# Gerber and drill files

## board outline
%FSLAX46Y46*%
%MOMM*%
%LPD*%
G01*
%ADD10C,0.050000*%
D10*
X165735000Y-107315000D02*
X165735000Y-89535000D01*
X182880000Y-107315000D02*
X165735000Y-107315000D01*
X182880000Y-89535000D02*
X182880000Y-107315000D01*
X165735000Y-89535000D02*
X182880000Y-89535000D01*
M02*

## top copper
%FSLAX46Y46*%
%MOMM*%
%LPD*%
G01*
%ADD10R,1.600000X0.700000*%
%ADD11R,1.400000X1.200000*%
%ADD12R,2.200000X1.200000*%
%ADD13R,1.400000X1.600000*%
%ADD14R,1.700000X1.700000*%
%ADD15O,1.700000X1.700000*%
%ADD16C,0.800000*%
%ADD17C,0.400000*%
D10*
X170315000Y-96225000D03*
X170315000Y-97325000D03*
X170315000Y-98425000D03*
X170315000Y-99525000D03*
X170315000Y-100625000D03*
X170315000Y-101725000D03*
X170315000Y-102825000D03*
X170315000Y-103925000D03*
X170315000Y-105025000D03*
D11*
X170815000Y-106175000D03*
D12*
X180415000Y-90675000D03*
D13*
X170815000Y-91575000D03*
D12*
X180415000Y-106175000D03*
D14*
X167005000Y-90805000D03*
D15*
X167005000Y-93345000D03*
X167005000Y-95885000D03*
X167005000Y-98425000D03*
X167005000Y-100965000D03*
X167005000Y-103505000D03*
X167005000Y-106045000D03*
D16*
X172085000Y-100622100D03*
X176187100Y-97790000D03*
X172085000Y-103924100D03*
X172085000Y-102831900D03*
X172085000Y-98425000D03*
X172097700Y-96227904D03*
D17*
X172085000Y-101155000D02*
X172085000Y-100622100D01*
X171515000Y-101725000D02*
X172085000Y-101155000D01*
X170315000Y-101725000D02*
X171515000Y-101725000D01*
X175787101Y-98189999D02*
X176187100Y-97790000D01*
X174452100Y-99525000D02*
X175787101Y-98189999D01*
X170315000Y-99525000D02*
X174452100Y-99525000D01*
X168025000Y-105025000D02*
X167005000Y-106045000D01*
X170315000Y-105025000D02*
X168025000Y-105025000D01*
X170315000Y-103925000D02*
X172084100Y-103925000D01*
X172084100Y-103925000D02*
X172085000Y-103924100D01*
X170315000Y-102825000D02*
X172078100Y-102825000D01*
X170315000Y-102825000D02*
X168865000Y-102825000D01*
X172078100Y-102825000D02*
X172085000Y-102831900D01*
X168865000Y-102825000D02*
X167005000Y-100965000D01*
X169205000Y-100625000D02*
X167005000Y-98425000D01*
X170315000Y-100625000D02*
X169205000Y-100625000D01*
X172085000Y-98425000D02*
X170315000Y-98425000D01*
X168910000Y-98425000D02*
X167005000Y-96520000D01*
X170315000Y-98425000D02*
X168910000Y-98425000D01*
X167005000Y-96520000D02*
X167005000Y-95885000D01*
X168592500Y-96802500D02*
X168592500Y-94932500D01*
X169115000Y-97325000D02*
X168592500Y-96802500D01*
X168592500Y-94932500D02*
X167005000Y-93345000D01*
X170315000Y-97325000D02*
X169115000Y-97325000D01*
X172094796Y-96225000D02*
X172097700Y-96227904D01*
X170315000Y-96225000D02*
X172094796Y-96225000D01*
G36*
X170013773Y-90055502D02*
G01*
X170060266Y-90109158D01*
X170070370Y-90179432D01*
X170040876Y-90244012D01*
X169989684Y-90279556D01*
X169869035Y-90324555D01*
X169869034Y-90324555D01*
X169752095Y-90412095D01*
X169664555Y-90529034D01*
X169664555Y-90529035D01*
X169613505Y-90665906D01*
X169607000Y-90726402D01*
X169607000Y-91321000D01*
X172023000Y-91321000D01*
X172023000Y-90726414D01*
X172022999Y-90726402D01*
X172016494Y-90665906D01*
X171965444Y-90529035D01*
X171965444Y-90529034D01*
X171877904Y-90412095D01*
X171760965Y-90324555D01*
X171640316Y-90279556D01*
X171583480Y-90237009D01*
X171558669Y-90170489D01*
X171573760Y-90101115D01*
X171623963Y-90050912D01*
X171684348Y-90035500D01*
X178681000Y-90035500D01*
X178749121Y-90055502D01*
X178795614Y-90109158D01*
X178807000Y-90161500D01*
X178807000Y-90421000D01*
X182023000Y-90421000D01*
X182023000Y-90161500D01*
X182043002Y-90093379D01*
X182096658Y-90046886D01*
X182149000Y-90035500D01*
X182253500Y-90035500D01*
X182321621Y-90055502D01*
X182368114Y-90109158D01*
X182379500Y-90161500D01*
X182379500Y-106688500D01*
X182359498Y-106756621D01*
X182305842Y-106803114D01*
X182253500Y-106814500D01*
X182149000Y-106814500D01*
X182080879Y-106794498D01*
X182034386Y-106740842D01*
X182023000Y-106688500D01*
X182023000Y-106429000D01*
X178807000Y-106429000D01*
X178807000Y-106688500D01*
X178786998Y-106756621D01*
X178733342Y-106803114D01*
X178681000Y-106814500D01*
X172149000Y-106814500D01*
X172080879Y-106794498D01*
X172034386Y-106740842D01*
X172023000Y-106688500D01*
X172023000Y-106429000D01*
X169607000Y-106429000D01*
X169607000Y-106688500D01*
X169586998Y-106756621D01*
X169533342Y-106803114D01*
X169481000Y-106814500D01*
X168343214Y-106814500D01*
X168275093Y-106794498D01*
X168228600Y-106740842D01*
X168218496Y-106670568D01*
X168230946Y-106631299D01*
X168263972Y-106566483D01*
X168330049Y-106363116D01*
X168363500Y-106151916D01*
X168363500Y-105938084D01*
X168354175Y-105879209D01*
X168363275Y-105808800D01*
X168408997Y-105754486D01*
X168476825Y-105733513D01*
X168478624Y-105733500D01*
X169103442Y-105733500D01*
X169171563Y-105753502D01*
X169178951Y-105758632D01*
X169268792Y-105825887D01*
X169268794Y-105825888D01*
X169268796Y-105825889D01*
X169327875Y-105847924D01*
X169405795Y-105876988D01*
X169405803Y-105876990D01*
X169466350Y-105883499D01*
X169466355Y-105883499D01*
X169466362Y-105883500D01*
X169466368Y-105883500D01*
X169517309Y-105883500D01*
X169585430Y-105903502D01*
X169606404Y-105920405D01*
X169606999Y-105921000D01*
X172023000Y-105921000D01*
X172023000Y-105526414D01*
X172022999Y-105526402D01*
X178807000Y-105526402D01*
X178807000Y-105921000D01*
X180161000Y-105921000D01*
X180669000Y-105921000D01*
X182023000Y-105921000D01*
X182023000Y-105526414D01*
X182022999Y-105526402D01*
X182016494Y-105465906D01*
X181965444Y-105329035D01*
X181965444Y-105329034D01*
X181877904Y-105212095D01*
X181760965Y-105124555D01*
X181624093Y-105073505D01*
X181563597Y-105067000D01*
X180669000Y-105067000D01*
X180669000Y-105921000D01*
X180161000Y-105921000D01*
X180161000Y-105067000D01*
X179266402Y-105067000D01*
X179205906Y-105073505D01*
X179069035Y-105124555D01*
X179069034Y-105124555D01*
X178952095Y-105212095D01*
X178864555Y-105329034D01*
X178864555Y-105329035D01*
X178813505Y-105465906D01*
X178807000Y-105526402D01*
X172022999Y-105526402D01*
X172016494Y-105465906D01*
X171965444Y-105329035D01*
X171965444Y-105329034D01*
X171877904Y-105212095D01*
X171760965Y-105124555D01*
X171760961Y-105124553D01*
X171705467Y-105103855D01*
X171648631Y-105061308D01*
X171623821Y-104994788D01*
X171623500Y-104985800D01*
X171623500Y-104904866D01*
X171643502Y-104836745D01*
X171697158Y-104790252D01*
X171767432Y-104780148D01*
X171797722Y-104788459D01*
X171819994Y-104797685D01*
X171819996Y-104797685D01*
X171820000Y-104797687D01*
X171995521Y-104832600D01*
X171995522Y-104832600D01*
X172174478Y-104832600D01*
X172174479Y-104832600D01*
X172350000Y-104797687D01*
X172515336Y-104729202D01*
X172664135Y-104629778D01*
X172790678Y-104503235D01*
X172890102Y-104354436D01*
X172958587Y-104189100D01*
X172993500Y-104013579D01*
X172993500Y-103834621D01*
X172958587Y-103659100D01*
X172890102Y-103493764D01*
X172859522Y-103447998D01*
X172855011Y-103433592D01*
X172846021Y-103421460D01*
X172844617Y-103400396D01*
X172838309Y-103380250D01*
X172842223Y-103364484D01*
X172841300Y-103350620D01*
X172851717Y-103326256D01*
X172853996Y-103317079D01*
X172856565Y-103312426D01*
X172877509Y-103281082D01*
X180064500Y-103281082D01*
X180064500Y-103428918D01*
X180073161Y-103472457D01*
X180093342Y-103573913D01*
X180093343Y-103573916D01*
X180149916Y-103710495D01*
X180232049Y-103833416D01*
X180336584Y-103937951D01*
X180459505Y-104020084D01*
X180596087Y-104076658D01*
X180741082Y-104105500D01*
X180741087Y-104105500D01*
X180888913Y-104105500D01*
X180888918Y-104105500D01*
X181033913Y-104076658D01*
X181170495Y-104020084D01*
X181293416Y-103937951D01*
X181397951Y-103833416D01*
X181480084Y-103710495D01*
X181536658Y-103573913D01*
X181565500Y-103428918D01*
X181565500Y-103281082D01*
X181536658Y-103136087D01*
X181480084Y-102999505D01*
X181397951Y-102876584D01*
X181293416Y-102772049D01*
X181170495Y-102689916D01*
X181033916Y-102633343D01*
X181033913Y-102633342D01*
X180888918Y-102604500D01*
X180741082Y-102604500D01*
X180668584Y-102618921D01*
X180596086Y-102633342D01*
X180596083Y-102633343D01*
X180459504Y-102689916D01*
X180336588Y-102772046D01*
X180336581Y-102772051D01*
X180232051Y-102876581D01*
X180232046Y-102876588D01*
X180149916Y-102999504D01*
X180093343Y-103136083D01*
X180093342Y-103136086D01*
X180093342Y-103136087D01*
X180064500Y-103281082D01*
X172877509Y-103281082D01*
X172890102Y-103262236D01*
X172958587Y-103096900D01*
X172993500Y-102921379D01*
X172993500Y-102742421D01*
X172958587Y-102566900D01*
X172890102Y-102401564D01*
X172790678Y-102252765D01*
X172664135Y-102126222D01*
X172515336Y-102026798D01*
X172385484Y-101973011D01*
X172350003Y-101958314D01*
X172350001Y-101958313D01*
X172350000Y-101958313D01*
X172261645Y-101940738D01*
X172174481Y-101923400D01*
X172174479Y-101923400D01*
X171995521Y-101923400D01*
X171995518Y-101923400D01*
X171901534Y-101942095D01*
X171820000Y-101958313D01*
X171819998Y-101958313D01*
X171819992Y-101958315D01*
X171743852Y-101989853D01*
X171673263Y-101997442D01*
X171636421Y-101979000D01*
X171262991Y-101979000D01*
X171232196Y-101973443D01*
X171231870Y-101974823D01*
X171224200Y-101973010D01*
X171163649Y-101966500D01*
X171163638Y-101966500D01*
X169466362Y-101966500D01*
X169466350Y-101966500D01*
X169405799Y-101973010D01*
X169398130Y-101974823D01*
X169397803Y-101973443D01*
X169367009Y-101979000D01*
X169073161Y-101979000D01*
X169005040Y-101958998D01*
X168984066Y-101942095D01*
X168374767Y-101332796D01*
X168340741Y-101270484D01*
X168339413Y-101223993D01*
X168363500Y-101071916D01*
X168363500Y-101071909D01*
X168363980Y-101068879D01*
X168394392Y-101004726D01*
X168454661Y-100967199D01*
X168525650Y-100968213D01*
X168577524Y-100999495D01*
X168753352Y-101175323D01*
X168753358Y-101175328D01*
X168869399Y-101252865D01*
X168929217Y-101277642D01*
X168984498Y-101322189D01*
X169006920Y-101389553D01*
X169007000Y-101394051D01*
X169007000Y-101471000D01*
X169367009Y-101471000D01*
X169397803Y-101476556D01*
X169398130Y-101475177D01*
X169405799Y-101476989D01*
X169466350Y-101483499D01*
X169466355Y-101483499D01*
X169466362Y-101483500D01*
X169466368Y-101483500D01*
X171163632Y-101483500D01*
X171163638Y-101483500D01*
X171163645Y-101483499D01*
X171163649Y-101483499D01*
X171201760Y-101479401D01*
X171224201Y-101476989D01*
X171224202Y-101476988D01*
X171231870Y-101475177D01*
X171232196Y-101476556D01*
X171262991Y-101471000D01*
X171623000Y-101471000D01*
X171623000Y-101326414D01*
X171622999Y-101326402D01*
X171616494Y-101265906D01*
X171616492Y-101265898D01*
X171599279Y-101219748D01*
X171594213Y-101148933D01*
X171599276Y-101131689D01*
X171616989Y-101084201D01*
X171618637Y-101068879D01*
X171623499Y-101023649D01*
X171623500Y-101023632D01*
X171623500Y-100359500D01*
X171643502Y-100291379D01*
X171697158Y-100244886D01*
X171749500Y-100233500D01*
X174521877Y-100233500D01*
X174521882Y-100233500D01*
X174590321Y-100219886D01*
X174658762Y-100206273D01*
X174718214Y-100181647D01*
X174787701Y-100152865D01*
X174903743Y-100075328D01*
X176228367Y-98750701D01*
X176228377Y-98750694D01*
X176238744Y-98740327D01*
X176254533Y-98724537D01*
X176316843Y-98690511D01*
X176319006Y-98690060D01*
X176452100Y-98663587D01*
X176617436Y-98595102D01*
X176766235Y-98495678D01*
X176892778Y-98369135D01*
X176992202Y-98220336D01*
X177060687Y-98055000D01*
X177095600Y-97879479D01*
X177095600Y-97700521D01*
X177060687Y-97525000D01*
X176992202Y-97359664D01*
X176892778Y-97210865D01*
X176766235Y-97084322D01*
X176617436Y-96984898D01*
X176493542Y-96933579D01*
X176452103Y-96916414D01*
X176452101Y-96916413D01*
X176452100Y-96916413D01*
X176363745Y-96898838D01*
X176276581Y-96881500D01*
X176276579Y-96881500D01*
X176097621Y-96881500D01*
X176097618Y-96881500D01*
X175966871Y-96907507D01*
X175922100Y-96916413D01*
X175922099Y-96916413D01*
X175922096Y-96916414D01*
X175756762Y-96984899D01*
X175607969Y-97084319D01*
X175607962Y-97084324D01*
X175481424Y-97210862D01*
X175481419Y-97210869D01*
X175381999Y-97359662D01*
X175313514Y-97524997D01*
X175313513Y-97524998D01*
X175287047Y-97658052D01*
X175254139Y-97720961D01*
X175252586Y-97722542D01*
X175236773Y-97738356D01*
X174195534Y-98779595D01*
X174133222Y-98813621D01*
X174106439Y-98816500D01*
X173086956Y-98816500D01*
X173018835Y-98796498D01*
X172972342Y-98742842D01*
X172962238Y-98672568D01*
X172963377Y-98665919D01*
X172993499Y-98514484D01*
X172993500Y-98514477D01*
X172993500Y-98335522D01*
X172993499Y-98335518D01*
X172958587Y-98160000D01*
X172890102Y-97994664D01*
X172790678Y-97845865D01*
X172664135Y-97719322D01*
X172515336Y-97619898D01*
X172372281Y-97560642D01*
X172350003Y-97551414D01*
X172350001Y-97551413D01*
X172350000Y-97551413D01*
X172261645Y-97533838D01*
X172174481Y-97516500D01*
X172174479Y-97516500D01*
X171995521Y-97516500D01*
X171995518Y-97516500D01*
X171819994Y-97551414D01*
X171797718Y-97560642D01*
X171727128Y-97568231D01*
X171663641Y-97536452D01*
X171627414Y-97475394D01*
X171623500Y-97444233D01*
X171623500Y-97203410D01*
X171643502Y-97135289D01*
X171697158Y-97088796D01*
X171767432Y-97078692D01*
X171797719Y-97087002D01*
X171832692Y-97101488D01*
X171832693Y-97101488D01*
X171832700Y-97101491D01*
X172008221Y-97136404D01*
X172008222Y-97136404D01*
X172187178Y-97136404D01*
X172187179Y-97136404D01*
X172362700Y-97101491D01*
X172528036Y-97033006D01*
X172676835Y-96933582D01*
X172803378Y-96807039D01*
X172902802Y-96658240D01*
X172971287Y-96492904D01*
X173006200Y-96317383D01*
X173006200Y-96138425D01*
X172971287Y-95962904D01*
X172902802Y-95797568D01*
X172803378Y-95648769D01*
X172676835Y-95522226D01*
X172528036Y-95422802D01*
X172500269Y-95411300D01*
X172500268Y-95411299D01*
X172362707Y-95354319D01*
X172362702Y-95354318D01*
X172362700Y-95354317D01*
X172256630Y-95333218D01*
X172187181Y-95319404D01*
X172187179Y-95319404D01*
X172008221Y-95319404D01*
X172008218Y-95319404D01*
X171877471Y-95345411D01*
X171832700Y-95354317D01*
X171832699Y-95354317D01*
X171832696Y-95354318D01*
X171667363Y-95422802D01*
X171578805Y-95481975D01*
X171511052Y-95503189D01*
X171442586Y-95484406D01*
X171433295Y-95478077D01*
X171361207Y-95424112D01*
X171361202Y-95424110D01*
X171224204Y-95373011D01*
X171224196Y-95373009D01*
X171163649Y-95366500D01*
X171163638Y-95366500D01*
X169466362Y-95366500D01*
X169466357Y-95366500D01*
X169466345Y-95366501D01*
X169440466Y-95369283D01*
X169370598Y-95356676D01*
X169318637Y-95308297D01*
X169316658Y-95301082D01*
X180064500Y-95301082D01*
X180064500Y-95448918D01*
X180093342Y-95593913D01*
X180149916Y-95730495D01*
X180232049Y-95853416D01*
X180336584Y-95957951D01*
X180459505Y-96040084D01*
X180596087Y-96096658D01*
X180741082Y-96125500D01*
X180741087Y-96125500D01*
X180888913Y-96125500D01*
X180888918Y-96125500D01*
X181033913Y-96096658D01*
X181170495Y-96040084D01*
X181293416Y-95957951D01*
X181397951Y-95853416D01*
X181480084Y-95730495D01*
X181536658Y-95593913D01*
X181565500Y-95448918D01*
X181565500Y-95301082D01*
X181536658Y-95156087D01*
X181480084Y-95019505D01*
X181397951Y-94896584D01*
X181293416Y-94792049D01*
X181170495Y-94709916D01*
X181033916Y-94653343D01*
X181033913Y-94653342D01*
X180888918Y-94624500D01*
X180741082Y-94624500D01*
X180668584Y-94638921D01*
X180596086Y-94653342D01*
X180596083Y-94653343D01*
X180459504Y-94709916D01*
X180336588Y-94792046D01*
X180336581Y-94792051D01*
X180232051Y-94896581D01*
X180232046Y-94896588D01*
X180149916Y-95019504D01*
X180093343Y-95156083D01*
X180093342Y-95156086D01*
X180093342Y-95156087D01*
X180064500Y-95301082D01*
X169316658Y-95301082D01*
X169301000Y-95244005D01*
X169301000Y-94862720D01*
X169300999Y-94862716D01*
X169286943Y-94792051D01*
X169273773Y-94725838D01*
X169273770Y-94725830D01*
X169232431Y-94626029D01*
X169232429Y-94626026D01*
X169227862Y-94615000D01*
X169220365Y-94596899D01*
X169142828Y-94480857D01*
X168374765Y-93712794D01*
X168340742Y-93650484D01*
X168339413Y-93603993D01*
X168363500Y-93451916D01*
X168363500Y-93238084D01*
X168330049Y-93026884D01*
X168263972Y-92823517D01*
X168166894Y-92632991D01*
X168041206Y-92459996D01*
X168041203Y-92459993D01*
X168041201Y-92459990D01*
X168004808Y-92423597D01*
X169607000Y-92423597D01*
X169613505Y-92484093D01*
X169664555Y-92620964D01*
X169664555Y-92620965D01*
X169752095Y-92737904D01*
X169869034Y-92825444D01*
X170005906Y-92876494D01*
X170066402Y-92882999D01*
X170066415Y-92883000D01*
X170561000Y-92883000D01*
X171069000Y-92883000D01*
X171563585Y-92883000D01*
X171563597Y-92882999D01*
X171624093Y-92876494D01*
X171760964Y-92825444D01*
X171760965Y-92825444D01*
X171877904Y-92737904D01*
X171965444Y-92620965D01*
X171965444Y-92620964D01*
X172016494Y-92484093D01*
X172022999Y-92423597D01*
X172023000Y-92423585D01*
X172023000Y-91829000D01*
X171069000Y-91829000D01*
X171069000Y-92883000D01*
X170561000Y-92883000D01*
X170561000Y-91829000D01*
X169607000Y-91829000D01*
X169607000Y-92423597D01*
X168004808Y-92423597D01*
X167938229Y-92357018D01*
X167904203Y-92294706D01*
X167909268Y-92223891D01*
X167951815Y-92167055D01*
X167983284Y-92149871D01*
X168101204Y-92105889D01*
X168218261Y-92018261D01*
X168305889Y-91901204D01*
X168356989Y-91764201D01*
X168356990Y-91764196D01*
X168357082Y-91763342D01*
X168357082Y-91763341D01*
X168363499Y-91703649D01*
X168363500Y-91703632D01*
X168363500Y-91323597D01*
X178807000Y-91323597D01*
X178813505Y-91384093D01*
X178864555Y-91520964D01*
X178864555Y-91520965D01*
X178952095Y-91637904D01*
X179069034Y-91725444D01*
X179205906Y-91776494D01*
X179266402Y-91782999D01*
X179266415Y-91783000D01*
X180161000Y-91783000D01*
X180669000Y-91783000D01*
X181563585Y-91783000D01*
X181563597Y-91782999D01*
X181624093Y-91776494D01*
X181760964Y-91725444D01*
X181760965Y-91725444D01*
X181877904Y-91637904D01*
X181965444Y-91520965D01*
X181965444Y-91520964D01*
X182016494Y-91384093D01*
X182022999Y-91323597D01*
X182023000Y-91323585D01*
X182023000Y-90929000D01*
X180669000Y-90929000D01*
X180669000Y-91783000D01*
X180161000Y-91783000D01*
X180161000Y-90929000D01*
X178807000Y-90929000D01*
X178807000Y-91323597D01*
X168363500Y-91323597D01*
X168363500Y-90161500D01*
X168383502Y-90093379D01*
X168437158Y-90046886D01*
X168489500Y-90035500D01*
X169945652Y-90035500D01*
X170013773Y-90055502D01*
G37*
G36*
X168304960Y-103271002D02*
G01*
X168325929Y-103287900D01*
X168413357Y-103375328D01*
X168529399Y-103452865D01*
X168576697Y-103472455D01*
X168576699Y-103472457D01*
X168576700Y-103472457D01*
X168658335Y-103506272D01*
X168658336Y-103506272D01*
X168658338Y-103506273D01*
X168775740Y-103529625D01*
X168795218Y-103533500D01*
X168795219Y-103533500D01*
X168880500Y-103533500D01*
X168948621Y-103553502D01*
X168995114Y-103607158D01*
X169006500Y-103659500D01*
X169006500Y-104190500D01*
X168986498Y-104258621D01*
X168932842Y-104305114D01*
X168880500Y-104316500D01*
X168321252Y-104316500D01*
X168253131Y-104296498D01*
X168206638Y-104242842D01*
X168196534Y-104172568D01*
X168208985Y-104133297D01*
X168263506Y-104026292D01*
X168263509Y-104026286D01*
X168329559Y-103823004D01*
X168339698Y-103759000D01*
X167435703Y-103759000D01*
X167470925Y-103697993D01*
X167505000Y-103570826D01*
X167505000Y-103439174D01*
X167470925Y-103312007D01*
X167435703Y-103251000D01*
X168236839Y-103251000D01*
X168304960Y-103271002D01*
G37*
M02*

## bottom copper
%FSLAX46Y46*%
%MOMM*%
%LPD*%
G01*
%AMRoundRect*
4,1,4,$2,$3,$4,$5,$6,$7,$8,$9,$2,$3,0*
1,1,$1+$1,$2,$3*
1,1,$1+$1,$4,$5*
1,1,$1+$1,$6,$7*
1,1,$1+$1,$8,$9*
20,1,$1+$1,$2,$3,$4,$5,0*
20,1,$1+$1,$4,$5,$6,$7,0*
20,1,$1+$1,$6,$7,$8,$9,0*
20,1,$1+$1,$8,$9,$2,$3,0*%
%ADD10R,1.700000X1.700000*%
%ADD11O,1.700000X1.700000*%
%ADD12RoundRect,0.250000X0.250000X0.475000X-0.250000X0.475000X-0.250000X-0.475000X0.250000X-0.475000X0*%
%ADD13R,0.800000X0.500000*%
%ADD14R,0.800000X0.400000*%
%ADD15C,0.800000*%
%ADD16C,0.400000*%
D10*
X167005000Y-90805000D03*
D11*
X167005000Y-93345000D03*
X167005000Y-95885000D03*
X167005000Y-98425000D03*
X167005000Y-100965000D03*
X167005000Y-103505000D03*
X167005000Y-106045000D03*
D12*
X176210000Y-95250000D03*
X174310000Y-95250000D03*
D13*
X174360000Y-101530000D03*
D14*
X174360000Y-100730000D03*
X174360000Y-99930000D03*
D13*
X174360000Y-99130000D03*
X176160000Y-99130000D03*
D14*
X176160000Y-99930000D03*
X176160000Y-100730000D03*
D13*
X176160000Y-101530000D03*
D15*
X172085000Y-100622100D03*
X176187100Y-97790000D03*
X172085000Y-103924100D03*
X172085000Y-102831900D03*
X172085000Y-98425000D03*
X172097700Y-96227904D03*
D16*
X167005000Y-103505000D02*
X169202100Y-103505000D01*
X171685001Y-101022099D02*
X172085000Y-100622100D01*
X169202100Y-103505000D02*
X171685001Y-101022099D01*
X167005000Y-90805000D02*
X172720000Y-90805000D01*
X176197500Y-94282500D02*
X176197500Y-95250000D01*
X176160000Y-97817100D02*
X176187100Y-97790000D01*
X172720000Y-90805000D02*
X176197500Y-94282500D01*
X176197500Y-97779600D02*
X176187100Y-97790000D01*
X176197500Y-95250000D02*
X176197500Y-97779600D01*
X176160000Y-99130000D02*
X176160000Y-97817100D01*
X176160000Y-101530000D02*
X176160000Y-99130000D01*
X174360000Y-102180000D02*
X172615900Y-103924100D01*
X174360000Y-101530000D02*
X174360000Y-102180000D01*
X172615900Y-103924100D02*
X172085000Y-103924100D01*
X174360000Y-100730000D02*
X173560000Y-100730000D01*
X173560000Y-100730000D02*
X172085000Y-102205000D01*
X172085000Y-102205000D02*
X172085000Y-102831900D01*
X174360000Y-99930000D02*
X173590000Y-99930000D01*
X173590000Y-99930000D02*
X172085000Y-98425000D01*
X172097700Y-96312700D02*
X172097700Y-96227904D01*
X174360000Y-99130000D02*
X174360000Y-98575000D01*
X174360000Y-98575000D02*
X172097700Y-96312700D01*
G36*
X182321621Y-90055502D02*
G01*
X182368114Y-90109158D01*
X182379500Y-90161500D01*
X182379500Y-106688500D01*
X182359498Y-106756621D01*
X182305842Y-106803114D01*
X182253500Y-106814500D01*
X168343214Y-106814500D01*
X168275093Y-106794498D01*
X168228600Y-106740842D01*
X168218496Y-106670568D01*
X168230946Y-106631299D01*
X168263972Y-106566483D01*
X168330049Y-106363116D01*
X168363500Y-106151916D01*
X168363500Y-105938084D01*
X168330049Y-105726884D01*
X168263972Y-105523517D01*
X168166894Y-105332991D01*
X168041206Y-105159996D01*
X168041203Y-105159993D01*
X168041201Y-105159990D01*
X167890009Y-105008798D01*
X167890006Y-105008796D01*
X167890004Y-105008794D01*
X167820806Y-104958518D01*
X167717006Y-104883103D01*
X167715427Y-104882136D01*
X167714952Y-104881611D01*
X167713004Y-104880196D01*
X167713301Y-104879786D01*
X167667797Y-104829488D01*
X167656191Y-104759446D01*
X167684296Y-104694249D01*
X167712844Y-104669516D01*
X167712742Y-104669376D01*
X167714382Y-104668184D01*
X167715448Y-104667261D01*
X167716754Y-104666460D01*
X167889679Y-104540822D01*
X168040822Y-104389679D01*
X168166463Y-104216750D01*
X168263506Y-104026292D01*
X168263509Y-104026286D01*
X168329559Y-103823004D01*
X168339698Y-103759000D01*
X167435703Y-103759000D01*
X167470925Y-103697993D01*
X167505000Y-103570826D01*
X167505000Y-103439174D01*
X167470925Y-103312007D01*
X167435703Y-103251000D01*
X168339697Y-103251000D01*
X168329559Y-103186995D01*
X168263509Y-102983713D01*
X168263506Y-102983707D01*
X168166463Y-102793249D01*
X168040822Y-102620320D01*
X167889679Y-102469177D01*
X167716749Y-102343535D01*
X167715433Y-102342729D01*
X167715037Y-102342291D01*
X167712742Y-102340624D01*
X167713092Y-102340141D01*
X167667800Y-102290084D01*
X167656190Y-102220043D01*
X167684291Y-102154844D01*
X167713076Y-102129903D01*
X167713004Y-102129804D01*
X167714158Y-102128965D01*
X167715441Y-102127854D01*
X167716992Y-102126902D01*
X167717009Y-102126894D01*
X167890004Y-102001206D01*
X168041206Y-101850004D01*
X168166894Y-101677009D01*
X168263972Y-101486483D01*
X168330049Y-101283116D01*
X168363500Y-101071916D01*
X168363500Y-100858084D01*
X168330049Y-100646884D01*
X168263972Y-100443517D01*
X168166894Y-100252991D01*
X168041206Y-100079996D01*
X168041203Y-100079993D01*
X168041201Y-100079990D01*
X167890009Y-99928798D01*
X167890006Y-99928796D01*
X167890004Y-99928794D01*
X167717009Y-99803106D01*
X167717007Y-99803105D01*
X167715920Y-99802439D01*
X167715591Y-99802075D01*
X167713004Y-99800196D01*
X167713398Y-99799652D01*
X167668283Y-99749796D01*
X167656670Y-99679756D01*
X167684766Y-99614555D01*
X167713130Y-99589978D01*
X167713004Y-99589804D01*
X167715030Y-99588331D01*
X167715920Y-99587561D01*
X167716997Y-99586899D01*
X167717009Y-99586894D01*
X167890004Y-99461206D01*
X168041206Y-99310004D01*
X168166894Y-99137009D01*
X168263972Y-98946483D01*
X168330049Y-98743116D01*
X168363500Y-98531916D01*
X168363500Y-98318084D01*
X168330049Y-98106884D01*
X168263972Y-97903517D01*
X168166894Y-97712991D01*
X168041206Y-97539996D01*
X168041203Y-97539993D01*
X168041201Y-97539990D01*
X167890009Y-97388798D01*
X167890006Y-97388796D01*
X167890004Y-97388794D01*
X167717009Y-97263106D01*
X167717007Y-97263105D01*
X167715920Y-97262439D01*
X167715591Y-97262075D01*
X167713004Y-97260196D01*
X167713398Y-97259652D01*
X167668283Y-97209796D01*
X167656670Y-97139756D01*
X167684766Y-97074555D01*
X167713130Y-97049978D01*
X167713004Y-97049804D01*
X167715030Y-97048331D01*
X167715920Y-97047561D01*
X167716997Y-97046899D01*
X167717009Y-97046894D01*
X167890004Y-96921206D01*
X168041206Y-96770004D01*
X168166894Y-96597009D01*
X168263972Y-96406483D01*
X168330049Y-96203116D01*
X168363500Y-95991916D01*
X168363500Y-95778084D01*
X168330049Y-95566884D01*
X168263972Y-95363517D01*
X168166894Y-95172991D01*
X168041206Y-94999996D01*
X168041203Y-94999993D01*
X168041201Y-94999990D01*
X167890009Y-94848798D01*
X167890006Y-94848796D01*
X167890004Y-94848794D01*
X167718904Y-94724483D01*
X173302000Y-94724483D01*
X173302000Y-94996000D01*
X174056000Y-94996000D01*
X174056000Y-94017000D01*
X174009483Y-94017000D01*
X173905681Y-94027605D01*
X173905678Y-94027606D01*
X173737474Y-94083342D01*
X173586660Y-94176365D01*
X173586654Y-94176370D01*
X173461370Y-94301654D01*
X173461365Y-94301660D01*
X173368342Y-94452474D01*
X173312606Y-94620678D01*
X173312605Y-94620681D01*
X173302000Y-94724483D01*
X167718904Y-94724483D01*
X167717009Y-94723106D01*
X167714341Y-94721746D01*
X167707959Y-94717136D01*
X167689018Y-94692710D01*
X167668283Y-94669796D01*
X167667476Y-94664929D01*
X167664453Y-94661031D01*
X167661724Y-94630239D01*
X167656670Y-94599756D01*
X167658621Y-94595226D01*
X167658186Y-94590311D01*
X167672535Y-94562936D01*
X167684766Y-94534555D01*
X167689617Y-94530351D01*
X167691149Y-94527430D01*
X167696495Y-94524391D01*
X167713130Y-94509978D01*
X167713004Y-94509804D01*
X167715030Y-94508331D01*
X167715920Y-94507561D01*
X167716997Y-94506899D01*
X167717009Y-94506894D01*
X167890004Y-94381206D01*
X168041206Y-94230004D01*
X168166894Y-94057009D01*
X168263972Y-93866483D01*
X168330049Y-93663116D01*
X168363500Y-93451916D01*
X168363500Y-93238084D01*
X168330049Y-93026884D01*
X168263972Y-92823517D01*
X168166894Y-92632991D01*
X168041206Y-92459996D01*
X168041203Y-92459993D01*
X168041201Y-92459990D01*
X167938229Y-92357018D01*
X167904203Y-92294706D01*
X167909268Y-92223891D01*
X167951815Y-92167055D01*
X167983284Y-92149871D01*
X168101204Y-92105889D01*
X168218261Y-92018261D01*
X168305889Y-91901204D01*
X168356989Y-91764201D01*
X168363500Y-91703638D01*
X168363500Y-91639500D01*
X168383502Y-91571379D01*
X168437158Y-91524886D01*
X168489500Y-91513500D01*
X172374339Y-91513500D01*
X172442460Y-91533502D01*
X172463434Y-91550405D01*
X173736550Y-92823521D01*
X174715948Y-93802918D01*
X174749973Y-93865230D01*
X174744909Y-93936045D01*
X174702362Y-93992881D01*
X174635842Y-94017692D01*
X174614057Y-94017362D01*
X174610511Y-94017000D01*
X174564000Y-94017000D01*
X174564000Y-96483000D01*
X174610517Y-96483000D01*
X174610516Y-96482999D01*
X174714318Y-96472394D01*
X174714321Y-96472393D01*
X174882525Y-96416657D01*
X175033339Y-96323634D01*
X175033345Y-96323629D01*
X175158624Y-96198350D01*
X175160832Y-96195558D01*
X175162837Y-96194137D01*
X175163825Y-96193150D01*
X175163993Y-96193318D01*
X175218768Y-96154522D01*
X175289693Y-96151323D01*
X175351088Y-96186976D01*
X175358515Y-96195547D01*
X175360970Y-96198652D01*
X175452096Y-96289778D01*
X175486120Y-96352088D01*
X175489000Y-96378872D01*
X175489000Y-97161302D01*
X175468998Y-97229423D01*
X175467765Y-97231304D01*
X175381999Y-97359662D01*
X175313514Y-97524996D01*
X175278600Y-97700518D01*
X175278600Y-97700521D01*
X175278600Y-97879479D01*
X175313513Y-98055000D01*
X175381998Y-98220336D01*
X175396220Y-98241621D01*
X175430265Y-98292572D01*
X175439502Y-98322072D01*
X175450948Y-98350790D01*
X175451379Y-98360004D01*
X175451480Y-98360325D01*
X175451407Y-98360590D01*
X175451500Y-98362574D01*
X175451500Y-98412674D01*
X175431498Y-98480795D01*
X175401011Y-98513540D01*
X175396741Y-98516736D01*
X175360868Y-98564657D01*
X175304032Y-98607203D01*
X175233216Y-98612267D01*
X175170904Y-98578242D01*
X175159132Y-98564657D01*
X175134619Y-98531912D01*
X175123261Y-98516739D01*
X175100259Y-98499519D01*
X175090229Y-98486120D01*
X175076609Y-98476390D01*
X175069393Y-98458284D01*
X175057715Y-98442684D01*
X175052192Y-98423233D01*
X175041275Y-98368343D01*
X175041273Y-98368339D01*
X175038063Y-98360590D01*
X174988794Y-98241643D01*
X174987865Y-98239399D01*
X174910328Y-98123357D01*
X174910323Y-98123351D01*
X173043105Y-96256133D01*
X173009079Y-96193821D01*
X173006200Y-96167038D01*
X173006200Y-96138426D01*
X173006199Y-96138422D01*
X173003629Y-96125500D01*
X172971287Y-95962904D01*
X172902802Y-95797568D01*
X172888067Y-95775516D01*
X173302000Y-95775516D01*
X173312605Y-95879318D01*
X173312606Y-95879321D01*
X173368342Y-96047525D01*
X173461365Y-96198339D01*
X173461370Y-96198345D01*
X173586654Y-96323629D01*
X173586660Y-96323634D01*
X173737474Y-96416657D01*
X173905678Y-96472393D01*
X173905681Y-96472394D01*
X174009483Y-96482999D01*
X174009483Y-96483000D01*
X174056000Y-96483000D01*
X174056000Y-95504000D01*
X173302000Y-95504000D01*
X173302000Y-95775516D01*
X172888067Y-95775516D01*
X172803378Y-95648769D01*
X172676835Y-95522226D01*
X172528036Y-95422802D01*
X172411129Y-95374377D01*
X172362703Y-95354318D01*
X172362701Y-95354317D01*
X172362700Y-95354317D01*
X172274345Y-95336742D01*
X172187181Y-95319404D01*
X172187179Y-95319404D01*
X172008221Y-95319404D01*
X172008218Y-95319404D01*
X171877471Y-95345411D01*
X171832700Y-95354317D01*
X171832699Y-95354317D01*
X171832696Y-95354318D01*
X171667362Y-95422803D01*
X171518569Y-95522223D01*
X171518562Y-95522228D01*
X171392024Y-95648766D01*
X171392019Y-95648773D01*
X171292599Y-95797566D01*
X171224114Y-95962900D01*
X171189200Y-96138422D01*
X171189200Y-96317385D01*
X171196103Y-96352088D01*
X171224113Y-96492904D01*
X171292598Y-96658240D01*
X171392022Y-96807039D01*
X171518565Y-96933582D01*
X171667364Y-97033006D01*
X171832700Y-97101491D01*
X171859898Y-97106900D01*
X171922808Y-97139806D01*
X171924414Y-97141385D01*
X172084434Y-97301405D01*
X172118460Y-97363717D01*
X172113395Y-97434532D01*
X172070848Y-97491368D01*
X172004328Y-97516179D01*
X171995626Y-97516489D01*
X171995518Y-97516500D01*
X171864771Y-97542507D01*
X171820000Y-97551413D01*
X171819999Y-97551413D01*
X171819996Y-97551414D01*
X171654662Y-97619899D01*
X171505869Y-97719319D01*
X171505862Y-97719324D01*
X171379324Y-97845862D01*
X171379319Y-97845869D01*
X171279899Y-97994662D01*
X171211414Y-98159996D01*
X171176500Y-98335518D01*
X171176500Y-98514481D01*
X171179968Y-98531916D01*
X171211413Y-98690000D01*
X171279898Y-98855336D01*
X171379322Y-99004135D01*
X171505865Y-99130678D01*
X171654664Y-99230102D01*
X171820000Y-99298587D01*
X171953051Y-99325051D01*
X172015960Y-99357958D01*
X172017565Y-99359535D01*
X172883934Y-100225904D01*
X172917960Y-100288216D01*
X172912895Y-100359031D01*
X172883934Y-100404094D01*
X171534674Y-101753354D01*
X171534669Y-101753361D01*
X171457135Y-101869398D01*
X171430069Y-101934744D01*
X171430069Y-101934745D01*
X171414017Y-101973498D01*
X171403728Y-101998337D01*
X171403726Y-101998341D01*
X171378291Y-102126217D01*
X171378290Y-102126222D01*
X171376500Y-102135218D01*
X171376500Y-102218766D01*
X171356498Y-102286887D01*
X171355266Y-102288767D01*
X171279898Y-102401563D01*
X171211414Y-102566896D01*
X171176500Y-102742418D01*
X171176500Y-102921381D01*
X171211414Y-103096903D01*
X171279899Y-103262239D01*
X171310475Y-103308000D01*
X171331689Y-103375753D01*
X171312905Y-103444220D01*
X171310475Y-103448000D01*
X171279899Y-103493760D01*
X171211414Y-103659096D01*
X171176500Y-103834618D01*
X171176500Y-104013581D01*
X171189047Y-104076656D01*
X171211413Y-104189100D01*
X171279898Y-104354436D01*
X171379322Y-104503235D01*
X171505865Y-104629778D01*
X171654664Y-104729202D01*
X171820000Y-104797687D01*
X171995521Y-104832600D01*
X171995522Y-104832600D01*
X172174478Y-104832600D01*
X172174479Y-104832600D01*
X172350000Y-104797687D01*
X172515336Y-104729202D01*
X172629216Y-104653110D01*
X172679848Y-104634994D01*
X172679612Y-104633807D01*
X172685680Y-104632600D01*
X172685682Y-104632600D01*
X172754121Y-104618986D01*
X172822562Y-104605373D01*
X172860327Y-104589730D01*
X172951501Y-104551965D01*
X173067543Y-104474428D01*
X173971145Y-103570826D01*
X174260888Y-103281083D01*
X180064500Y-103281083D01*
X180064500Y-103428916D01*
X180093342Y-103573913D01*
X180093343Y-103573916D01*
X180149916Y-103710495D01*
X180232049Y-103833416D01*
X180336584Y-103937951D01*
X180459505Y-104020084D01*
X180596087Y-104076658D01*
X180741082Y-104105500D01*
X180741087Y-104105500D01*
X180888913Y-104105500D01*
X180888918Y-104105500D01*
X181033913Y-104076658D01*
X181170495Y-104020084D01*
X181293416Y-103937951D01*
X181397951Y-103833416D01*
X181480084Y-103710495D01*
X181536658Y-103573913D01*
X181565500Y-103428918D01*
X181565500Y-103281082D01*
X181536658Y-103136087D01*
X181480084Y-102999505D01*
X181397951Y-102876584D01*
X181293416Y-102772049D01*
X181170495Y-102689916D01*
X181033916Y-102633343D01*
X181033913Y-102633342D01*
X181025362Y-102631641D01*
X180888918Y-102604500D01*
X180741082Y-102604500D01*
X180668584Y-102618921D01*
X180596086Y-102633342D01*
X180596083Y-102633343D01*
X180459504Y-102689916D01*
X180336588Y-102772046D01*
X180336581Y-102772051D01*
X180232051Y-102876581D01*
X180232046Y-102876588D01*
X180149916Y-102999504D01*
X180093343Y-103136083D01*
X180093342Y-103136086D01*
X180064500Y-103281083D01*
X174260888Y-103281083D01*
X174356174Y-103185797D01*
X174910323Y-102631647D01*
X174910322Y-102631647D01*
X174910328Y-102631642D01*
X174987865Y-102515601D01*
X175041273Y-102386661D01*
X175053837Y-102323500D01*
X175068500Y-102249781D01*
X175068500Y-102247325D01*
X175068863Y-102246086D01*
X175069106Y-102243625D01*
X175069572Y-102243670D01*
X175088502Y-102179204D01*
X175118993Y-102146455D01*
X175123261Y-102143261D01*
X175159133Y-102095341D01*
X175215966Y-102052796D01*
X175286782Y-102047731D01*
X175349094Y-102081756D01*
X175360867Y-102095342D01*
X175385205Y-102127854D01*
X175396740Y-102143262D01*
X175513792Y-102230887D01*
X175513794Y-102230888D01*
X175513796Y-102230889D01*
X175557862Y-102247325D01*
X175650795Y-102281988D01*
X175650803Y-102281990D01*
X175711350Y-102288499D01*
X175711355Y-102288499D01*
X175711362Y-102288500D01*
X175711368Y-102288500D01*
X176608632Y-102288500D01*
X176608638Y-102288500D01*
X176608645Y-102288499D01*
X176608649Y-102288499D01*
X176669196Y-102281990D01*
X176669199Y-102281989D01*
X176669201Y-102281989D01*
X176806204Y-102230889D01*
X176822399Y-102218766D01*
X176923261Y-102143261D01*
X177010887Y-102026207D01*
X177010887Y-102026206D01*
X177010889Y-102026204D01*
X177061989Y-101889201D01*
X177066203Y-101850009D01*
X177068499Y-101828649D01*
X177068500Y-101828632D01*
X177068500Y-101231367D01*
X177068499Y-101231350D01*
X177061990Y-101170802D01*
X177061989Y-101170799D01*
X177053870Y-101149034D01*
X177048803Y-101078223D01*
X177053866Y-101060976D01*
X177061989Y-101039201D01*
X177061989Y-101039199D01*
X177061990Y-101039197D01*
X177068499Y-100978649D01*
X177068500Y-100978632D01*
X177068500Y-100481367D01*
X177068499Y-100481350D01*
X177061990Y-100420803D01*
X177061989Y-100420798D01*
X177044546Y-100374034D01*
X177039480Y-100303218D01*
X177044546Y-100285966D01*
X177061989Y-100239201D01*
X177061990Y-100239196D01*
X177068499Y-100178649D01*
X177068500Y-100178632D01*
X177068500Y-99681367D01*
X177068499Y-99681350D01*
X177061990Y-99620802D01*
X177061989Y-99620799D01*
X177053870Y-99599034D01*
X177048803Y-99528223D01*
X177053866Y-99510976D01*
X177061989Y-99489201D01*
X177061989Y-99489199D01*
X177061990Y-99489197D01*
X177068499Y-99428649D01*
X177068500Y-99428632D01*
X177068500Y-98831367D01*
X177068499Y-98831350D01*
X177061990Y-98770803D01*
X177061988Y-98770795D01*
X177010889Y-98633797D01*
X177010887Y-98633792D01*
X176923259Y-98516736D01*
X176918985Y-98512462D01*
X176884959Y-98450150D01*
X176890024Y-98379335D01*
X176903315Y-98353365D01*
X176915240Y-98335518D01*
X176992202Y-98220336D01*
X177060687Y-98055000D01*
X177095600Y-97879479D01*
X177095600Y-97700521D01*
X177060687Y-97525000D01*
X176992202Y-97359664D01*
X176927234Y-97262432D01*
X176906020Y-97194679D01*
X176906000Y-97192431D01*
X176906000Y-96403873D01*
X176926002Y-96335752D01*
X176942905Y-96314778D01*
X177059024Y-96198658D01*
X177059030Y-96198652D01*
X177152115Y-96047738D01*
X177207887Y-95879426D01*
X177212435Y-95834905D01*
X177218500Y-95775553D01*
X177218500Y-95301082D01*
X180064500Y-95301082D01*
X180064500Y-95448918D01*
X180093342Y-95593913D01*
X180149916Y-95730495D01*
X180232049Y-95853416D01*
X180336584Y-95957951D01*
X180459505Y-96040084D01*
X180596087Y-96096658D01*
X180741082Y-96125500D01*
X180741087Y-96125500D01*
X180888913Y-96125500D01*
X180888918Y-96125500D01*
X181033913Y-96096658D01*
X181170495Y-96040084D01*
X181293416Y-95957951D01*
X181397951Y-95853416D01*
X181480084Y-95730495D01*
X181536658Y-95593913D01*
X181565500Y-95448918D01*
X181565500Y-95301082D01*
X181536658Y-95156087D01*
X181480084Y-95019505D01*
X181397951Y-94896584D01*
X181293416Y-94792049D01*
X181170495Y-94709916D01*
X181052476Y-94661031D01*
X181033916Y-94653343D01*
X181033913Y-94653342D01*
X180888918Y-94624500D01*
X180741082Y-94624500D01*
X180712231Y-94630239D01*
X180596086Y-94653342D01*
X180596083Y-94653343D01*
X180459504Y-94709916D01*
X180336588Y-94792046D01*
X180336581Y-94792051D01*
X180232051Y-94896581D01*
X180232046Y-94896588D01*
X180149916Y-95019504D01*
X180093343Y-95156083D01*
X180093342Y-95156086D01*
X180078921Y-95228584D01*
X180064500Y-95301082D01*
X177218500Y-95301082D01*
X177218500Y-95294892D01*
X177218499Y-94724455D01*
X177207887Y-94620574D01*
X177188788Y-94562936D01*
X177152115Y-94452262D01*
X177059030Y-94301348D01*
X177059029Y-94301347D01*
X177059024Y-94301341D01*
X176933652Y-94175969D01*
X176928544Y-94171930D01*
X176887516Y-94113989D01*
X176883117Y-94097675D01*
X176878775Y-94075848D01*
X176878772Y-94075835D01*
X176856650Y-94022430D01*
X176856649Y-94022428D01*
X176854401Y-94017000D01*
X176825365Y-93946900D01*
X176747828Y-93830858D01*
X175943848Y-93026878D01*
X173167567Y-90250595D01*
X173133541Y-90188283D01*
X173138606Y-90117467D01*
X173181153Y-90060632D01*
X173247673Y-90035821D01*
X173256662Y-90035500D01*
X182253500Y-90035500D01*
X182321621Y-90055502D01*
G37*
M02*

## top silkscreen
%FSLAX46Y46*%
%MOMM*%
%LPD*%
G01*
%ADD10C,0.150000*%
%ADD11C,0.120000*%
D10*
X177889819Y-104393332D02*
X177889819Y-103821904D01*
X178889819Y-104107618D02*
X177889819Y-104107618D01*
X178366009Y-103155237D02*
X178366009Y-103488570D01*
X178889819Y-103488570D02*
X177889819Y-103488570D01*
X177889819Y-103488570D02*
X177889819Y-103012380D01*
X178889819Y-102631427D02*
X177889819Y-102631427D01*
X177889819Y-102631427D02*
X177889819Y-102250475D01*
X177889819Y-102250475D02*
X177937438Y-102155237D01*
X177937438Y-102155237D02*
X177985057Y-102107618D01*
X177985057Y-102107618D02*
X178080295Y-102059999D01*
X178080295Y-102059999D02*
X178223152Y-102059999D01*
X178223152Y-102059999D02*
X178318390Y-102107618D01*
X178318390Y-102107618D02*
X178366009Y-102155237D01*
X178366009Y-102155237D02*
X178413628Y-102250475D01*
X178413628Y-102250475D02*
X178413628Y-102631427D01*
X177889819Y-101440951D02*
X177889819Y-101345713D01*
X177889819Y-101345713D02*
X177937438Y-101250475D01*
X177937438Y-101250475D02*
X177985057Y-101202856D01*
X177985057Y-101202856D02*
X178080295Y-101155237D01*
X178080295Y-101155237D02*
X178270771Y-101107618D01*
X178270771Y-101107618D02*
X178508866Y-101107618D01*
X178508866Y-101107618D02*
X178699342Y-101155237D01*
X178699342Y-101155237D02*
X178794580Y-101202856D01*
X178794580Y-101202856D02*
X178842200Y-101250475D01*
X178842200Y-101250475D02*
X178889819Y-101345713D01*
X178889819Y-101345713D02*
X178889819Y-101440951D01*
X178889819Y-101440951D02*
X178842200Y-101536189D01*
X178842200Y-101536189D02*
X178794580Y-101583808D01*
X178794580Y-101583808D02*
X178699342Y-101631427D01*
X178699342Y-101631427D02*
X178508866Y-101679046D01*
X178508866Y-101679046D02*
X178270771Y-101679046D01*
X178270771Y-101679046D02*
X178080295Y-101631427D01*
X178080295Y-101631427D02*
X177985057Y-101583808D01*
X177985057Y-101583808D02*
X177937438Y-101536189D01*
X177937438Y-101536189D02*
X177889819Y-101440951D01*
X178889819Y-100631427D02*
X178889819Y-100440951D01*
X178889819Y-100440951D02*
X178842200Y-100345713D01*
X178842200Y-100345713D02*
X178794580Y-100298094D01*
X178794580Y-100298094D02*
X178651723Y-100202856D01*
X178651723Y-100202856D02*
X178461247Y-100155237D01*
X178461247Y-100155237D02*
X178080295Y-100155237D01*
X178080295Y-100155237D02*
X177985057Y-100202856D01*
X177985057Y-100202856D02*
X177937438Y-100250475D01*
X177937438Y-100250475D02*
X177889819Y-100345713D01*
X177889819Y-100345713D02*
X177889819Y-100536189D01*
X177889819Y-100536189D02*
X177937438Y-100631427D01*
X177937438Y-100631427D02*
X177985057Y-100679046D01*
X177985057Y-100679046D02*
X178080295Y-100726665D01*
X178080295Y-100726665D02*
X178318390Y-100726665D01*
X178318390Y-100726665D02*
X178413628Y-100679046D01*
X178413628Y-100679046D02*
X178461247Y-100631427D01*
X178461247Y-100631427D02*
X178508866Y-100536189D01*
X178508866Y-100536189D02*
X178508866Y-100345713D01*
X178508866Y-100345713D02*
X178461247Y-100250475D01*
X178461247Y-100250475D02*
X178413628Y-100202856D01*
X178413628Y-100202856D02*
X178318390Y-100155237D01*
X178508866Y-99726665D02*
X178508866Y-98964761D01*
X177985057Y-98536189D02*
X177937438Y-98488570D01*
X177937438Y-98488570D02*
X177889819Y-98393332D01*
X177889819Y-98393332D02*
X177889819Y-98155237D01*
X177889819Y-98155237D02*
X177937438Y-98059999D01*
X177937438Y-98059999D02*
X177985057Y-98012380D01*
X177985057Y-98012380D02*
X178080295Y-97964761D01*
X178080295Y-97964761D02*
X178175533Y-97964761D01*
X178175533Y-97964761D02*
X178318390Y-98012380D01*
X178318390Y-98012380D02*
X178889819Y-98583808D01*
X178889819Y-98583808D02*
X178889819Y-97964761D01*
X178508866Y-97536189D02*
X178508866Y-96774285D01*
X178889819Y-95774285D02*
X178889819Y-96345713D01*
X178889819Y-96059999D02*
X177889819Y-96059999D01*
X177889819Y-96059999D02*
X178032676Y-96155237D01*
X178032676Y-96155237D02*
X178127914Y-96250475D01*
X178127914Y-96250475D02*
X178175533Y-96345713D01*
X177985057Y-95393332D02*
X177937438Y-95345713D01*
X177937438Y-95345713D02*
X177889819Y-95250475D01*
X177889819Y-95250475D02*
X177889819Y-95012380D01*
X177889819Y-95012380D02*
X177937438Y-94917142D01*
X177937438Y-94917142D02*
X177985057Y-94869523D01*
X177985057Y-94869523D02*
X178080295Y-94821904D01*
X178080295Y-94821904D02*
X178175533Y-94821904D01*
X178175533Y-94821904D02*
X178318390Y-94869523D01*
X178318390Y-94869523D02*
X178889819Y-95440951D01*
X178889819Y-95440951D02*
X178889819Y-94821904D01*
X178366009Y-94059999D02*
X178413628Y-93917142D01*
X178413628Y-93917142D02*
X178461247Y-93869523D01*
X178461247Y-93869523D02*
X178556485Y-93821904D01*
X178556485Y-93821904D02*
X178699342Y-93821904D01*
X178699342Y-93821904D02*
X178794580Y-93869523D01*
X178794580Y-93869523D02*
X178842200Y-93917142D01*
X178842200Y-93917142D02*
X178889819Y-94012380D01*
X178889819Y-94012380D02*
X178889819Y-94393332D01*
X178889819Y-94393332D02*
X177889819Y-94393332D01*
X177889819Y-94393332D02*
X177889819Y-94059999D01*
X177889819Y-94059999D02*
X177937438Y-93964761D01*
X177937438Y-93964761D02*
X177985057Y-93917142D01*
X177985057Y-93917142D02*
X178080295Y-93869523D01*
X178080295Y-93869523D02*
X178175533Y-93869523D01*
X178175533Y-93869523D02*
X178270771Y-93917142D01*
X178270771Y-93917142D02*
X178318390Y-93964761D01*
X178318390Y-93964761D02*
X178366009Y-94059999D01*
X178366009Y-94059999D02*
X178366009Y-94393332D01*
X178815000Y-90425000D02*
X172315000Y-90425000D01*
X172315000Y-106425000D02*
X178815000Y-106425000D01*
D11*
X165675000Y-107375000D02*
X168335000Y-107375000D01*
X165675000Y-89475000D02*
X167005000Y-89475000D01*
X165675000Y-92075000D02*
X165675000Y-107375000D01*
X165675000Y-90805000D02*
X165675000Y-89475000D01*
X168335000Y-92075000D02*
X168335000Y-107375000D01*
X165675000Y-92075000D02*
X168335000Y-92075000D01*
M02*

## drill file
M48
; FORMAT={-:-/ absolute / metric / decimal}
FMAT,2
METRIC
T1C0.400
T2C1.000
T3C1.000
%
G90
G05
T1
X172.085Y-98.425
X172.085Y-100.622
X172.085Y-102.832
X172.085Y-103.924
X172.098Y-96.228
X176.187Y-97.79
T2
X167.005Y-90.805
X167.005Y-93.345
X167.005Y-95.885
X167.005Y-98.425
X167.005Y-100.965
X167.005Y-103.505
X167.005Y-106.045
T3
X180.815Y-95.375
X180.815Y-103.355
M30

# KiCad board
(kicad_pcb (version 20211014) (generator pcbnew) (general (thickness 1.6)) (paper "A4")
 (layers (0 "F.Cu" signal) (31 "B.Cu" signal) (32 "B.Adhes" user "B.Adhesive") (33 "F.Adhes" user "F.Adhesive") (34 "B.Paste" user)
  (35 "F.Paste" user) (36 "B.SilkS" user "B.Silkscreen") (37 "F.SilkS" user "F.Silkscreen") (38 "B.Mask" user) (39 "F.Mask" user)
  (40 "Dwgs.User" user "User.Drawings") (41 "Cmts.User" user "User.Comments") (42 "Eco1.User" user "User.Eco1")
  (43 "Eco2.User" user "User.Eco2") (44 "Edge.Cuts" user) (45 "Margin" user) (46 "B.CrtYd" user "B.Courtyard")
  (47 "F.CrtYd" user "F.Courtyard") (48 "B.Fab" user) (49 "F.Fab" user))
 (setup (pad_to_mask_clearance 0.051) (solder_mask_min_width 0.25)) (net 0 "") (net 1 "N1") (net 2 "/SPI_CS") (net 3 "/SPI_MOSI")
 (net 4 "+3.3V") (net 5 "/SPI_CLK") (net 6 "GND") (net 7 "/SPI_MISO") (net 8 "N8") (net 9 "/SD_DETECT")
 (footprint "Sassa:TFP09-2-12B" (layer "F.Cu") (at 170.815 98.425 90)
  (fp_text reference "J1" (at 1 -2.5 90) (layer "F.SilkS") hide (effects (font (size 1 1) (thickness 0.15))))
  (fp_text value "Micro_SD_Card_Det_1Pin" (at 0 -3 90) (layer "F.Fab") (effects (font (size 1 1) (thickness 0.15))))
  (fp_line (start 8 8) (end 8 1.5) (layer "F.SilkS") (width 0.15))
  (fp_line (start -8 1.5) (end -8 8) (layer "F.SilkS") (width 0.15))
  (pad "" np_thru_hole circle locked (at -4.93 10 90) (size 1 1) (drill 1) (layers *.Cu *.Mask))
  (pad "" np_thru_hole circle locked (at 3.05 10 90) (size 1 1) (drill 1) (layers *.Cu *.Mask))
  (pad "1" smd rect locked (at 2.2 -0.5 90) (size 0.7 1.6) (layers "F.Cu" "F.Paste" "F.Mask") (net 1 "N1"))
  (pad "2" smd rect locked (at 1.1 -0.5 90) (size 0.7 1.6) (layers "F.Cu" "F.Paste" "F.Mask") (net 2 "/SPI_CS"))
  (pad "3" smd rect locked (at 0 -0.5 90) (size 0.7 1.6) (layers "F.Cu" "F.Paste" "F.Mask") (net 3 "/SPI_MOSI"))
  (pad "4" smd rect locked (at -1.1 -0.5 90) (size 0.7 1.6) (layers "F.Cu" "F.Paste" "F.Mask") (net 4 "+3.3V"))
  (pad "5" smd rect locked (at -2.2 -0.5 90) (size 0.7 1.6) (layers "F.Cu" "F.Paste" "F.Mask") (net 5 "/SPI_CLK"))
  (pad "6" smd rect locked (at -3.3 -0.5 90) (size 0.7 1.6) (layers "F.Cu" "F.Paste" "F.Mask") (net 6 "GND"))
  (pad "7" smd rect locked (at -4.4 -0.5 90) (size 0.7 1.6) (layers "F.Cu" "F.Paste" "F.Mask") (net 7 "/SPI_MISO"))
  (pad "8" smd rect locked (at -5.5 -0.5 90) (size 0.7 1.6) (layers "F.Cu" "F.Paste" "F.Mask") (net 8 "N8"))
  (pad "9" smd rect locked (at -6.6 -0.5 90) (size 0.7 1.6) (layers "F.Cu" "F.Paste" "F.Mask") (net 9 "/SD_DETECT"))
  (pad "10" smd rect locked (at -7.75 0 90) (size 1.2 1.4) (layers "F.Cu" "F.Paste" "F.Mask") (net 6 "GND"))
  (pad "10" smd rect locked (at 7.75 9.6 90) (size 1.2 2.2) (layers "F.Cu" "F.Paste" "F.Mask") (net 6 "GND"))
  (pad "10" smd rect locked (at 6.85 0 90) (size 1.6 1.4) (layers "F.Cu" "F.Paste" "F.Mask") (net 6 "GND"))
  (pad "10" smd rect locked (at -7.75 9.6 90) (size 1.2 2.2) (layers "F.Cu" "F.Paste" "F.Mask") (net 6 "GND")))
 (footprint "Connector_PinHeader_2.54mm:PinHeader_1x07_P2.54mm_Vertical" (layer "F.Cu") (at 167.005 90.805)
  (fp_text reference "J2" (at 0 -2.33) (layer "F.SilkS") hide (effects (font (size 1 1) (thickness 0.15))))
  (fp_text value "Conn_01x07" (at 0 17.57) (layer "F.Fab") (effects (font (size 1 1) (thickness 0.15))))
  (fp_line (start -1.33 16.57) (end 1.33 16.57) (layer "F.SilkS") (width 0.12))
  (fp_line (start -1.33 -1.33) (end 0 -1.33) (layer "F.SilkS") (width 0.12))
  (fp_line (start -1.33 1.27) (end -1.33 16.57) (layer "F.SilkS") (width 0.12))
  (fp_line (start -1.33 0) (end -1.33 -1.33) (layer "F.SilkS") (width 0.12))
  (fp_line (start 1.33 1.27) (end 1.33 16.57) (layer "F.SilkS") (width 0.12))
  (fp_line (start -1.33 1.27) (end 1.33 1.27) (layer "F.SilkS") (width 0.12))
  (pad "1" thru_hole rect (at 0 0) (size 1.7 1.7) (drill 1) (layers *.Cu *.Mask) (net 4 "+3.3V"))
  (pad "2" thru_hole oval (at 0 2.54) (size 1.7 1.7) (drill 1) (layers *.Cu *.Mask) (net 2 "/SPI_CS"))
  (pad "3" thru_hole oval (at 0 5.08) (size 1.7 1.7) (drill 1) (layers *.Cu *.Mask) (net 3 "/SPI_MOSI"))
  (pad "4" thru_hole oval (at 0 7.62) (size 1.7 1.7) (drill 1) (layers *.Cu *.Mask) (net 5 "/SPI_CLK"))
  (pad "5" thru_hole oval (at 0 10.16) (size 1.7 1.7) (drill 1) (layers *.Cu *.Mask) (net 7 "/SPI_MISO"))
  (pad "6" thru_hole oval (at 0 12.7) (size 1.7 1.7) (drill 1) (layers *.Cu *.Mask) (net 6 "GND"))
  (pad "7" thru_hole oval (at 0 15.24) (size 1.7 1.7) (drill 1) (layers *.Cu *.Mask) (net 9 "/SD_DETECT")))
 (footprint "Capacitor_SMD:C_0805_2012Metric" (layer "B.Cu") (at 175.26 95.25 180)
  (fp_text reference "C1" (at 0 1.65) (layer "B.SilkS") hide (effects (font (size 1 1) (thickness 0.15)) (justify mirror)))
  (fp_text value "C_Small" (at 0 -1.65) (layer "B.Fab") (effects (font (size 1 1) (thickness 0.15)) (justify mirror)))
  (pad "1" smd roundrect (at -0.95 0 180) (size 1 1.45) (layers "B.Cu" "B.Paste" "B.Mask") (roundrect_rratio 0.25) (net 4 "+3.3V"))
  (pad "2" smd roundrect (at 0.95 0 180) (size 1 1.45) (layers "B.Cu" "B.Paste" "B.Mask") (roundrect_rratio 0.25) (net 6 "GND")))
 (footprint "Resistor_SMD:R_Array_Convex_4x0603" (layer "B.Cu") (at 175.26 100.33)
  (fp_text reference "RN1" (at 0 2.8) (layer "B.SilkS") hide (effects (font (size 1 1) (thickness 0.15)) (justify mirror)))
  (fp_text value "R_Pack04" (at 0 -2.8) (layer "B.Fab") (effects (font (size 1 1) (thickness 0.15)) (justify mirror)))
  (pad "1" smd rect (at -0.9 1.2) (size 0.8 0.5) (layers "B.Cu" "B.Paste" "B.Mask") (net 8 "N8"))
  (pad "2" smd rect (at -0.9 0.4) (size 0.8 0.4) (layers "B.Cu" "B.Paste" "B.Mask") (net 7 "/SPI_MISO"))
  (pad "3" smd rect (at -0.9 -0.4) (size 0.8 0.4) (layers "B.Cu" "B.Paste" "B.Mask") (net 3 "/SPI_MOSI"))
  (pad "4" smd rect (at -0.9 -1.2) (size 0.8 0.5) (layers "B.Cu" "B.Paste" "B.Mask") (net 1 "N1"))
  (pad "5" smd rect (at 0.9 -1.2) (size 0.8 0.5) (layers "B.Cu" "B.Paste" "B.Mask") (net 4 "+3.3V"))
  (pad "6" smd rect (at 0.9 -0.4) (size 0.8 0.4) (layers "B.Cu" "B.Paste" "B.Mask") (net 4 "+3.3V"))
  (pad "7" smd rect (at 0.9 0.4) (size 0.8 0.4) (layers "B.Cu" "B.Paste" "B.Mask") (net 4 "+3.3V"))
  (pad "8" smd rect (at 0.9 1.2) (size 0.8 0.5) (layers "B.Cu" "B.Paste" "B.Mask") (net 4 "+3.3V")))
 (gr_line (start 165.735 107.315) (end 165.735 89.535) (layer "Edge.Cuts") (width 0.05))
 (gr_line (start 182.88 107.315) (end 165.735 107.315) (layer "Edge.Cuts") (width 0.05))
 (gr_line (start 182.88 89.535) (end 182.88 107.315) (layer "Edge.Cuts") (width 0.05))
 (gr_line (start 165.735 89.535) (end 182.88 89.535) (layer "Edge.Cuts") (width 0.05))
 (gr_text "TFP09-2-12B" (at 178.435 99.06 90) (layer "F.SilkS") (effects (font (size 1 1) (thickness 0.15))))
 (segment (start 172.085 101.155) (end 172.085 100.6221) (width 0.4) (layer "F.Cu") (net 6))
 (segment (start 171.515 101.725) (end 172.085 101.155) (width 0.4) (layer "F.Cu") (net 6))
 (segment (start 170.315 101.725) (end 171.515 101.725) (width 0.4) (layer "F.Cu") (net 6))
 (via (at 172.085 100.6221) (size 0.8) (drill 0.4) (layers "F.Cu" "B.Cu") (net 6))
 (segment (start 167.005 103.505) (end 169.2021 103.505) (width 0.4) (layer "B.Cu") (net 6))
 (segment (start 171.685001 101.022099) (end 172.085 100.6221) (width 0.4) (layer "B.Cu") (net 6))
 (segment (start 169.2021 103.505) (end 171.685001 101.022099) (width 0.4) (layer "B.Cu") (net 6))
 (segment (start 175.787101 98.189999) (end 176.1871 97.79) (width 0.4) (layer "F.Cu") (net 4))
 (segment (start 174.4521 99.525) (end 175.787101 98.189999) (width 0.4) (layer "F.Cu") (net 4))
 (segment (start 170.315 99.525) (end 174.4521 99.525) (width 0.4) (layer "F.Cu") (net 4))
 (via (at 176.1871 97.79) (size 0.8) (drill 0.4) (layers "F.Cu" "B.Cu") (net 4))
 (segment (start 167.005 90.805) (end 172.72 90.805) (width 0.4) (layer "B.Cu") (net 4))
 (segment (start 176.1975 94.2825) (end 176.1975 95.25) (width 0.4) (layer "B.Cu") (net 4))
 (segment (start 176.16 97.8171) (end 176.1871 97.79) (width 0.4) (layer "B.Cu") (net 4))
 (segment (start 172.72 90.805) (end 176.1975 94.2825) (width 0.4) (layer "B.Cu") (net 4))
 (segment (start 176.1975 97.7796) (end 176.1871 97.79) (width 0.4) (layer "B.Cu") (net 4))
 (segment (start 176.1975 95.25) (end 176.1975 97.7796) (width 0.4) (layer "B.Cu") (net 4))
 (segment (start 176.16 99.13) (end 176.16 97.8171) (width 0.4) (layer "B.Cu") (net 4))
 (segment (start 176.16 101.53) (end 176.16 99.13) (width 0.4) (layer "B.Cu") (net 4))
 (segment (start 168.025 105.025) (end 167.005 106.045) (width 0.4) (layer "F.Cu") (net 9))
 (segment (start 170.315 105.025) (end 168.025 105.025) (width 0.4) (layer "F.Cu") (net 9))
 (segment (start 170.315 103.925) (end 172.0841 103.925) (width 0.4) (layer "F.Cu") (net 8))
 (segment (start 172.0841 103.925) (end 172.085 103.9241) (width 0.4) (layer "F.Cu") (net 8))
 (via (at 172.085 103.9241) (size 0.8) (drill 0.4) (layers "F.Cu" "B.Cu") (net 8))
 (segment (start 174.36 102.18) (end 172.6159 103.9241) (width 0.4) (layer "B.Cu") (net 8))
 (segment (start 174.36 101.53) (end 174.36 102.18) (width 0.4) (layer "B.Cu") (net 8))
 (segment (start 172.6159 103.9241) (end 172.085 103.9241) (width 0.4) (layer "B.Cu") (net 8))
 (segment (start 170.315 102.825) (end 172.0781 102.825) (width 0.4) (layer "F.Cu") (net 7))
 (segment (start 170.315 102.825) (end 168.865 102.825) (width 0.4) (layer "F.Cu") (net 7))
 (segment (start 172.0781 102.825) (end 172.085 102.8319) (width 0.4) (layer "F.Cu") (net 7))
 (segment (start 168.865 102.825) (end 167.005 100.965) (width 0.4) (layer "F.Cu") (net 7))
 (via (at 172.085 102.8319) (size 0.8) (drill 0.4) (layers "F.Cu" "B.Cu") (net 7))
 (segment (start 174.36 100.73) (end 173.56 100.73) (width 0.4) (layer "B.Cu") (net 7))
 (segment (start 173.56 100.73) (end 172.085 102.205) (width 0.4) (layer "B.Cu") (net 7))
 (segment (start 172.085 102.205) (end 172.085 102.8319) (width 0.4) (layer "B.Cu") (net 7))
 (segment (start 169.205 100.625) (end 167.005 98.425) (width 0.4) (layer "F.Cu") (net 5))
 (segment (start 170.315 100.625) (end 169.205 100.625) (width 0.4) (layer "F.Cu") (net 5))
 (segment (start 172.085 98.425) (end 170.315 98.425) (width 0.4) (layer "F.Cu") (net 3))
 (segment (start 168.91 98.425) (end 167.005 96.52) (width 0.4) (layer "F.Cu") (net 3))
 (segment (start 170.315 98.425) (end 168.91 98.425) (width 0.4) (layer "F.Cu") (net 3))
 (segment (start 167.005 96.52) (end 167.005 95.885) (width 0.4) (layer "F.Cu") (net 3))
 (via (at 172.085 98.425) (size 0.8) (drill 0.4) (layers "F.Cu" "B.Cu") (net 3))
 (segment (start 174.36 99.93) (end 173.59 99.93) (width 0.4) (layer "B.Cu") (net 3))
 (segment (start 173.59 99.93) (end 172.085 98.425) (width 0.4) (layer "B.Cu") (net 3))
 (segment (start 168.5925 96.8025) (end 168.5925 94.9325) (width 0.4) (layer "F.Cu") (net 2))
 (segment (start 169.115 97.325) (end 168.5925 96.8025) (width 0.4) (layer "F.Cu") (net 2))
 (segment (start 168.5925 94.9325) (end 167.005 93.345) (width 0.4) (layer "F.Cu") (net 2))
 (segment (start 170.315 97.325) (end 169.115 97.325) (width 0.4) (layer "F.Cu") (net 2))
 (segment (start 172.094796 96.225) (end 172.0977 96.227904) (width 0.4) (layer "F.Cu") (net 1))
 (segment (start 170.315 96.225) (end 172.094796 96.225) (width 0.4) (layer "F.Cu") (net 1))
 (via (at 172.0977 96.227904) (size 0.8) (drill 0.4) (layers "F.Cu" "B.Cu") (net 1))
 (segment (start 172.0977 96.3127) (end 172.0977 96.227904) (width 0.4) (layer "B.Cu") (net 1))
 (segment (start 174.36 99.13) (end 174.36 98.575) (width 0.4) (layer "B.Cu") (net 1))
 (segment (start 174.36 98.575) (end 172.0977 96.3127) (width 0.4) (layer "B.Cu") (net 1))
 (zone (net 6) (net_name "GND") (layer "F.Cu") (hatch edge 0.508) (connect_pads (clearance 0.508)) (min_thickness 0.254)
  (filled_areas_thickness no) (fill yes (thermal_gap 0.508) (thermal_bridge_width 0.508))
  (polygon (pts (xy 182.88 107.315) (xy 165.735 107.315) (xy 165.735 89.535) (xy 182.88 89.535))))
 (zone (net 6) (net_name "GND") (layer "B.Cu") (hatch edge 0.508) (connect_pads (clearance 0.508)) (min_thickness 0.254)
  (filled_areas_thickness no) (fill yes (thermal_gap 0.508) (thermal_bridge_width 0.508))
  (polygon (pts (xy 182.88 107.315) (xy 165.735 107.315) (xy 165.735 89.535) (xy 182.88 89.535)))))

